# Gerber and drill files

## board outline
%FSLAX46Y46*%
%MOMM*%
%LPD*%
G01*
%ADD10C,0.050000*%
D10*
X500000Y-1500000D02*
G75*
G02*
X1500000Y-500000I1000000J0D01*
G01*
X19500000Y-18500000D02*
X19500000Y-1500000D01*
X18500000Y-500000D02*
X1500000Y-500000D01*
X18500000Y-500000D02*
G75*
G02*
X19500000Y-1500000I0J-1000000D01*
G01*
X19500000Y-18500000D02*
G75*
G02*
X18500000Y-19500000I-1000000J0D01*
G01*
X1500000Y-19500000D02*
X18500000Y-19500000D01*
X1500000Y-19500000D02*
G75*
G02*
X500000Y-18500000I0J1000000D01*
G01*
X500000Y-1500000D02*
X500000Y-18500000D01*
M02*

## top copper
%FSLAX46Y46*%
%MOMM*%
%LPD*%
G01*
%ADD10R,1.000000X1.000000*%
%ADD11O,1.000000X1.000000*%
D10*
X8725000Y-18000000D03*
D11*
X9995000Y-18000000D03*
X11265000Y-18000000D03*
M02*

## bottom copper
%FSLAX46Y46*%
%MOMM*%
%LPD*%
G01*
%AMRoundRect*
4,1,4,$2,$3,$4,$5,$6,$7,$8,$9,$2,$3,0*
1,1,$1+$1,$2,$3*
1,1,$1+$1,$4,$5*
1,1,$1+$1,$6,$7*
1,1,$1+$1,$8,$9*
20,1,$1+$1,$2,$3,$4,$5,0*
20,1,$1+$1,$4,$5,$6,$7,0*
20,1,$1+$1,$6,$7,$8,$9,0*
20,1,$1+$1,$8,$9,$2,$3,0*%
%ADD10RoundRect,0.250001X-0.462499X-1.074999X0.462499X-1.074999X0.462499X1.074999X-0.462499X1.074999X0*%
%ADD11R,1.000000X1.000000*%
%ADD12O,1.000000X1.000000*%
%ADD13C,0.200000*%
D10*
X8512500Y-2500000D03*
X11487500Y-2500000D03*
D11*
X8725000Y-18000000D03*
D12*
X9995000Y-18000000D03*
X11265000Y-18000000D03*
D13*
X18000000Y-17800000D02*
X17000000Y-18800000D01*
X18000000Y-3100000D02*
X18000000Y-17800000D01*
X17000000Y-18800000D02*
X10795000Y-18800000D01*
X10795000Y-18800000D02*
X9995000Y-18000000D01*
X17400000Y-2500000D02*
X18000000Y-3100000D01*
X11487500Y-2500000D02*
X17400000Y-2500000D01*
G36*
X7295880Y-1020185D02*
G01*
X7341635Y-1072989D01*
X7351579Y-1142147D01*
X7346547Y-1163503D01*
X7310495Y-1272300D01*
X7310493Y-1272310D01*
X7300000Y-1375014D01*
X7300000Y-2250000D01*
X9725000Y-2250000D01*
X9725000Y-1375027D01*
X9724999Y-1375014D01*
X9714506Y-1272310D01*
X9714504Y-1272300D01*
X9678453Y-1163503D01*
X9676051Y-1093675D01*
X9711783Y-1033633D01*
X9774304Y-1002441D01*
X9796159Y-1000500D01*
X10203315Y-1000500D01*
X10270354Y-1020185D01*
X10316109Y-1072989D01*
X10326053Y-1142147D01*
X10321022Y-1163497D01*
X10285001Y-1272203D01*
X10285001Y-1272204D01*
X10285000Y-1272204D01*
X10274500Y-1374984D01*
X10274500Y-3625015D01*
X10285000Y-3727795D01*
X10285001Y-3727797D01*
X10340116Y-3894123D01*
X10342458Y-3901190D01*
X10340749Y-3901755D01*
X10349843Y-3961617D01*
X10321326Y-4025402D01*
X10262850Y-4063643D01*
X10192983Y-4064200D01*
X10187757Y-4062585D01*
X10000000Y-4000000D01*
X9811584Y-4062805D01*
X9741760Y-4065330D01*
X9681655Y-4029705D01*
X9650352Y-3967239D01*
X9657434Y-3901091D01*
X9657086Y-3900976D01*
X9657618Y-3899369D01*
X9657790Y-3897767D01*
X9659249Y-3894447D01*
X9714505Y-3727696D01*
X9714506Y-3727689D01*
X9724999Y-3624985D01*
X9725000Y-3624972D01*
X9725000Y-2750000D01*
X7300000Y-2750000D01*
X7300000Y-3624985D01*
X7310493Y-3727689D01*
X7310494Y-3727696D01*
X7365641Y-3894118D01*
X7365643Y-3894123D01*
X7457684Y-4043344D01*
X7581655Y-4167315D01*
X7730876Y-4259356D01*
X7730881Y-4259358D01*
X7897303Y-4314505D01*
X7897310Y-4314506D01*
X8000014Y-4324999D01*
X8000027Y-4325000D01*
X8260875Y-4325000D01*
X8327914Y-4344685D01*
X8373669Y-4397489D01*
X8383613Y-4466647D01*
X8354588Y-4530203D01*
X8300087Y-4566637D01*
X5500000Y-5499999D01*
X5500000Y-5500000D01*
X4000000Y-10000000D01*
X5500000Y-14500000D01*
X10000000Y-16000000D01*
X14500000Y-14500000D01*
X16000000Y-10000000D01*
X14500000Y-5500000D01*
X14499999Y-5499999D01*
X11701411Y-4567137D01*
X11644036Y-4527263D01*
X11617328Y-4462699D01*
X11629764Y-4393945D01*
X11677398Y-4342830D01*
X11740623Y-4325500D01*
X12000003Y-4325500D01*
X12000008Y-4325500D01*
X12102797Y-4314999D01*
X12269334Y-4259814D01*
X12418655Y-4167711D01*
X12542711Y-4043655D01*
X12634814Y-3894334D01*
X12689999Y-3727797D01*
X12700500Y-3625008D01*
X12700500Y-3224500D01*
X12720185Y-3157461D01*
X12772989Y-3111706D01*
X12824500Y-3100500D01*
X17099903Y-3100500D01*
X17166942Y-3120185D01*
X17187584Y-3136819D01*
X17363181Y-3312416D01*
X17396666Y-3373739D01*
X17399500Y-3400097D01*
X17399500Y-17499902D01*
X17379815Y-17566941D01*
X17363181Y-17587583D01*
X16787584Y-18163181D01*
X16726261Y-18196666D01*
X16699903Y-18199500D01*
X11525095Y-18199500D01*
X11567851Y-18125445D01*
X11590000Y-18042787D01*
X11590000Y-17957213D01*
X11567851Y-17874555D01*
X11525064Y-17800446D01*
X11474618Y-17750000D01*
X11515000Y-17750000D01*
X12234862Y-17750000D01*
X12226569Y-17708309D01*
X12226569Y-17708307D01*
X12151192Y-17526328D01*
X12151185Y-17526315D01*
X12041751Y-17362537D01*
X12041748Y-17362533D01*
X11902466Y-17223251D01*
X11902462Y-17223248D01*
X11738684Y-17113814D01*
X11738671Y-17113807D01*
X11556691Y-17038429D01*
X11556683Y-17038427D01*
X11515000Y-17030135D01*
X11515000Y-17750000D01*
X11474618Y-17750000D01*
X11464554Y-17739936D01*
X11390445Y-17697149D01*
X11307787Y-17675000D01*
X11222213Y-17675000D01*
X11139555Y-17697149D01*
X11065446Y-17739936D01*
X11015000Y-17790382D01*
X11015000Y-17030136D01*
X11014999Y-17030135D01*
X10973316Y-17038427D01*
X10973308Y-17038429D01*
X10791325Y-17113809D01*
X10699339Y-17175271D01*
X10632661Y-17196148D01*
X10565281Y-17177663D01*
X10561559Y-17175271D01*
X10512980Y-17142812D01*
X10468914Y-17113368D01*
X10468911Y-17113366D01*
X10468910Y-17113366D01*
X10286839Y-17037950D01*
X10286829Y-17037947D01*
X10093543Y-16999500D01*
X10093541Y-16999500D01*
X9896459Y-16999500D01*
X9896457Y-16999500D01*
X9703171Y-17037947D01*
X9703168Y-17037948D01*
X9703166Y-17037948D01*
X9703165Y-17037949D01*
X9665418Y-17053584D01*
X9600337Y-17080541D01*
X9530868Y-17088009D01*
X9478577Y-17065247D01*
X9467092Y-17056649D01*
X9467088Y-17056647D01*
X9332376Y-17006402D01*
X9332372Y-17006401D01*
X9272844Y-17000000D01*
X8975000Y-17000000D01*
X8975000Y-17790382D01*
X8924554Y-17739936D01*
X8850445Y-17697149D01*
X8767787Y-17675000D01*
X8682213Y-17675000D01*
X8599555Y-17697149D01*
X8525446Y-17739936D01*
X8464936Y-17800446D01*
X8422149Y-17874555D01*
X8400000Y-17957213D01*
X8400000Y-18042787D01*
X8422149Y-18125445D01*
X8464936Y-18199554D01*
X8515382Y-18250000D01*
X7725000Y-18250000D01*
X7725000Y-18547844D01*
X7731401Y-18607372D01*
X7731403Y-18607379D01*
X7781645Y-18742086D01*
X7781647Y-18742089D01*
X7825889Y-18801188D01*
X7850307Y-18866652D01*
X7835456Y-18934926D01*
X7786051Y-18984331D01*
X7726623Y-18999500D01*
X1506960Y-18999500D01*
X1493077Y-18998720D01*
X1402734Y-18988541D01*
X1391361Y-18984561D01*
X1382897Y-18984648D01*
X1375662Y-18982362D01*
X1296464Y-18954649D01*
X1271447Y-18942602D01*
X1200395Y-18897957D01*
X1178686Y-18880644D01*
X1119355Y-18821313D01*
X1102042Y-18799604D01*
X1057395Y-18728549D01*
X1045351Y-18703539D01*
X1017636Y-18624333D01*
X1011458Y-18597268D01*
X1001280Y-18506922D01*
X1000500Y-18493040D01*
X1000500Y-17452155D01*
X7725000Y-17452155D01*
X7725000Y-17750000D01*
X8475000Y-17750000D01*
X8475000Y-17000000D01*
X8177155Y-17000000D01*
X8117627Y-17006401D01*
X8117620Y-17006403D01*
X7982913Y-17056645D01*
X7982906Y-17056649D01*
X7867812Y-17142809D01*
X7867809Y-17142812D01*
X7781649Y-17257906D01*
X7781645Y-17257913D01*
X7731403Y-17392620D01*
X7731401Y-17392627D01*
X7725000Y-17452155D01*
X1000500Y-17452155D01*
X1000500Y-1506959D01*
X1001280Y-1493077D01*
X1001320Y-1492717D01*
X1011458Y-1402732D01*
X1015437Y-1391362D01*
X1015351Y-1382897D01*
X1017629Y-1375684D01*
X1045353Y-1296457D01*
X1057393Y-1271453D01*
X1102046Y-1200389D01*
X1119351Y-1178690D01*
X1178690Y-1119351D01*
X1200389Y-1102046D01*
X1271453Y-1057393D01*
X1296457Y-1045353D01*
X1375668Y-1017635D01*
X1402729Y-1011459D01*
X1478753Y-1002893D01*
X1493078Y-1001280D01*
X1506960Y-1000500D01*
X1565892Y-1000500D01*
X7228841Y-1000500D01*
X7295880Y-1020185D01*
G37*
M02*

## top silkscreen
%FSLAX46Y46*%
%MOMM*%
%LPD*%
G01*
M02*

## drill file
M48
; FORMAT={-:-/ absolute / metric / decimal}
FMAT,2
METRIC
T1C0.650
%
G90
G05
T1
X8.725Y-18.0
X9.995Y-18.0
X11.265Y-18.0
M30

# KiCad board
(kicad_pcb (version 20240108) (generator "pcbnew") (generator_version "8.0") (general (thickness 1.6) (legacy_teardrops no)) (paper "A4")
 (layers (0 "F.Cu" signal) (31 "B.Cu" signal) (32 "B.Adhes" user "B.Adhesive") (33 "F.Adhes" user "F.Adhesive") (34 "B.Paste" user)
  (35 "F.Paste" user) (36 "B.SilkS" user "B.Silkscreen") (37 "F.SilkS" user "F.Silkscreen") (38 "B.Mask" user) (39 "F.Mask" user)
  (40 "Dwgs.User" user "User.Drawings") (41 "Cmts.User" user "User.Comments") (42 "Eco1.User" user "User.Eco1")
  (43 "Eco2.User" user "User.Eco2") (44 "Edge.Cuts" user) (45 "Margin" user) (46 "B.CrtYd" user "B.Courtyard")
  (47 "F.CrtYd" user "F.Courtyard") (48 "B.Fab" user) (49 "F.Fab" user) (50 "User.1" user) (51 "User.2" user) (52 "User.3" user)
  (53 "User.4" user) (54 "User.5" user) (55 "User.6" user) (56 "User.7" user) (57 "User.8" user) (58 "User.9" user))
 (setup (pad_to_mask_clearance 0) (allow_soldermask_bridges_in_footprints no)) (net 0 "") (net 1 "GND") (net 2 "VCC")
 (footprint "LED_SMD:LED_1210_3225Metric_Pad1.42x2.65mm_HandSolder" (layer "B.Cu") (at 10 2.5)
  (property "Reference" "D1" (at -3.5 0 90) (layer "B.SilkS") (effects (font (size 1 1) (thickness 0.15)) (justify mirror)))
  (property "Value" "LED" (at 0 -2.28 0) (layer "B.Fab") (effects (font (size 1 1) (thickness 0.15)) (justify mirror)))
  (pad "1" smd roundrect (at -1.4875 0) (size 1.425 2.65) (layers "B.Cu" "B.Paste" "B.Mask") (roundrect_rratio 0.175439) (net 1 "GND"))
  (pad "2" smd roundrect (at 1.4875 0) (size 1.425 2.65) (layers "B.Cu" "B.Paste" "B.Mask") (roundrect_rratio 0.175439) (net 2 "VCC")))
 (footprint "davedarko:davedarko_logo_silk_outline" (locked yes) (layer "B.Cu") (at 3.5 16 180)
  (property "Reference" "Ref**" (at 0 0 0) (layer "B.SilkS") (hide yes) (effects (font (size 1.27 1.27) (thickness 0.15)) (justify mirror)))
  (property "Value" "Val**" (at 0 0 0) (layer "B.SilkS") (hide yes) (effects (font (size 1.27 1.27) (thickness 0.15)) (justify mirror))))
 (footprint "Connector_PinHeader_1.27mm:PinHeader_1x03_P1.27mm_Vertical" (layer "B.Cu") (at 8.725 18 -90)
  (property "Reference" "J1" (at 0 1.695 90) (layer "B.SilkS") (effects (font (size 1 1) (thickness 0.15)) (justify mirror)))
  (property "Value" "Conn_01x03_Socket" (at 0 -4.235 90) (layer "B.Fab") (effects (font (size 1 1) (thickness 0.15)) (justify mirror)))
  (pad "1" thru_hole rect (at 0 0 270) (size 1 1) (drill 0.65) (layers "*.Cu" "*.Mask") (remove_unused_layers no) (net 1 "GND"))
  (pad "2" thru_hole oval (at 0 -1.27 270) (size 1 1) (drill 0.65) (layers "*.Cu" "*.Mask") (remove_unused_layers no) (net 2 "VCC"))
  (pad "3" thru_hole oval (at 0 -2.54 270) (size 1 1) (drill 0.65) (layers "*.Cu" "*.Mask") (remove_unused_layers no) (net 1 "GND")))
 (gr_arc (start 0.5 1.5) (mid 0.792893 0.792893) (end 1.5 0.5) (stroke (width 0.05) (type default)) (layer "Edge.Cuts"))
 (gr_line (start 19.5 18.5) (end 19.5 1.5) (stroke (width 0.05) (type default)) (layer "Edge.Cuts"))
 (gr_line (start 18.5 0.5) (end 1.5 0.5) (stroke (width 0.05) (type default)) (layer "Edge.Cuts"))
 (gr_arc (start 18.5 0.5) (mid 19.207107 0.792893) (end 19.5 1.5) (stroke (width 0.05) (type default)) (layer "Edge.Cuts"))
 (gr_arc (start 19.5 18.5) (mid 19.207107 19.207107) (end 18.5 19.5) (stroke (width 0.05) (type default)) (layer "Edge.Cuts"))
 (gr_line (start 1.5 19.5) (end 18.5 19.5) (stroke (width 0.05) (type default)) (layer "Edge.Cuts"))
 (gr_arc (start 1.5 19.5) (mid 0.792893 19.207107) (end 0.5 18.5) (stroke (width 0.05) (type default)) (layer "Edge.Cuts"))
 (gr_line (start 0.5 1.5) (end 0.5 18.5) (stroke (width 0.05) (type default)) (layer "Edge.Cuts"))
 (segment (start 18 17.8) (end 17 18.8) (width 0.2) (layer "B.Cu") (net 2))
 (segment (start 18 3.1) (end 18 17.8) (width 0.2) (layer "B.Cu") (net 2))
 (segment (start 17 18.8) (end 10.795 18.8) (width 0.2) (layer "B.Cu") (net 2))
 (segment (start 10.795 18.8) (end 9.995 18) (width 0.2) (layer "B.Cu") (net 2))
 (segment (start 17.4 2.5) (end 18 3.1) (width 0.2) (layer "B.Cu") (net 2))
 (segment (start 11.4875 2.5) (end 17.4 2.5) (width 0.2) (layer "B.Cu") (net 2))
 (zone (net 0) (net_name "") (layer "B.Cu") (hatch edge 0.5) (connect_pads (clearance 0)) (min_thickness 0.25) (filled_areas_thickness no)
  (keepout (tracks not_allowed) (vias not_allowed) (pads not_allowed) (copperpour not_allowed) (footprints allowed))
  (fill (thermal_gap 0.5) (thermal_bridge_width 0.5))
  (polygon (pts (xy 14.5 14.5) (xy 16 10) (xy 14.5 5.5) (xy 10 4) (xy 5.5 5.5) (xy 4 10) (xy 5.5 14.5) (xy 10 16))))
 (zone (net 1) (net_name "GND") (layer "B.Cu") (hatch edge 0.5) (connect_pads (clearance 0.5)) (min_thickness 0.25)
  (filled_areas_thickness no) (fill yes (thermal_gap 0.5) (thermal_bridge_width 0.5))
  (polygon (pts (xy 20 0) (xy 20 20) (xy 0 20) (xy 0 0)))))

